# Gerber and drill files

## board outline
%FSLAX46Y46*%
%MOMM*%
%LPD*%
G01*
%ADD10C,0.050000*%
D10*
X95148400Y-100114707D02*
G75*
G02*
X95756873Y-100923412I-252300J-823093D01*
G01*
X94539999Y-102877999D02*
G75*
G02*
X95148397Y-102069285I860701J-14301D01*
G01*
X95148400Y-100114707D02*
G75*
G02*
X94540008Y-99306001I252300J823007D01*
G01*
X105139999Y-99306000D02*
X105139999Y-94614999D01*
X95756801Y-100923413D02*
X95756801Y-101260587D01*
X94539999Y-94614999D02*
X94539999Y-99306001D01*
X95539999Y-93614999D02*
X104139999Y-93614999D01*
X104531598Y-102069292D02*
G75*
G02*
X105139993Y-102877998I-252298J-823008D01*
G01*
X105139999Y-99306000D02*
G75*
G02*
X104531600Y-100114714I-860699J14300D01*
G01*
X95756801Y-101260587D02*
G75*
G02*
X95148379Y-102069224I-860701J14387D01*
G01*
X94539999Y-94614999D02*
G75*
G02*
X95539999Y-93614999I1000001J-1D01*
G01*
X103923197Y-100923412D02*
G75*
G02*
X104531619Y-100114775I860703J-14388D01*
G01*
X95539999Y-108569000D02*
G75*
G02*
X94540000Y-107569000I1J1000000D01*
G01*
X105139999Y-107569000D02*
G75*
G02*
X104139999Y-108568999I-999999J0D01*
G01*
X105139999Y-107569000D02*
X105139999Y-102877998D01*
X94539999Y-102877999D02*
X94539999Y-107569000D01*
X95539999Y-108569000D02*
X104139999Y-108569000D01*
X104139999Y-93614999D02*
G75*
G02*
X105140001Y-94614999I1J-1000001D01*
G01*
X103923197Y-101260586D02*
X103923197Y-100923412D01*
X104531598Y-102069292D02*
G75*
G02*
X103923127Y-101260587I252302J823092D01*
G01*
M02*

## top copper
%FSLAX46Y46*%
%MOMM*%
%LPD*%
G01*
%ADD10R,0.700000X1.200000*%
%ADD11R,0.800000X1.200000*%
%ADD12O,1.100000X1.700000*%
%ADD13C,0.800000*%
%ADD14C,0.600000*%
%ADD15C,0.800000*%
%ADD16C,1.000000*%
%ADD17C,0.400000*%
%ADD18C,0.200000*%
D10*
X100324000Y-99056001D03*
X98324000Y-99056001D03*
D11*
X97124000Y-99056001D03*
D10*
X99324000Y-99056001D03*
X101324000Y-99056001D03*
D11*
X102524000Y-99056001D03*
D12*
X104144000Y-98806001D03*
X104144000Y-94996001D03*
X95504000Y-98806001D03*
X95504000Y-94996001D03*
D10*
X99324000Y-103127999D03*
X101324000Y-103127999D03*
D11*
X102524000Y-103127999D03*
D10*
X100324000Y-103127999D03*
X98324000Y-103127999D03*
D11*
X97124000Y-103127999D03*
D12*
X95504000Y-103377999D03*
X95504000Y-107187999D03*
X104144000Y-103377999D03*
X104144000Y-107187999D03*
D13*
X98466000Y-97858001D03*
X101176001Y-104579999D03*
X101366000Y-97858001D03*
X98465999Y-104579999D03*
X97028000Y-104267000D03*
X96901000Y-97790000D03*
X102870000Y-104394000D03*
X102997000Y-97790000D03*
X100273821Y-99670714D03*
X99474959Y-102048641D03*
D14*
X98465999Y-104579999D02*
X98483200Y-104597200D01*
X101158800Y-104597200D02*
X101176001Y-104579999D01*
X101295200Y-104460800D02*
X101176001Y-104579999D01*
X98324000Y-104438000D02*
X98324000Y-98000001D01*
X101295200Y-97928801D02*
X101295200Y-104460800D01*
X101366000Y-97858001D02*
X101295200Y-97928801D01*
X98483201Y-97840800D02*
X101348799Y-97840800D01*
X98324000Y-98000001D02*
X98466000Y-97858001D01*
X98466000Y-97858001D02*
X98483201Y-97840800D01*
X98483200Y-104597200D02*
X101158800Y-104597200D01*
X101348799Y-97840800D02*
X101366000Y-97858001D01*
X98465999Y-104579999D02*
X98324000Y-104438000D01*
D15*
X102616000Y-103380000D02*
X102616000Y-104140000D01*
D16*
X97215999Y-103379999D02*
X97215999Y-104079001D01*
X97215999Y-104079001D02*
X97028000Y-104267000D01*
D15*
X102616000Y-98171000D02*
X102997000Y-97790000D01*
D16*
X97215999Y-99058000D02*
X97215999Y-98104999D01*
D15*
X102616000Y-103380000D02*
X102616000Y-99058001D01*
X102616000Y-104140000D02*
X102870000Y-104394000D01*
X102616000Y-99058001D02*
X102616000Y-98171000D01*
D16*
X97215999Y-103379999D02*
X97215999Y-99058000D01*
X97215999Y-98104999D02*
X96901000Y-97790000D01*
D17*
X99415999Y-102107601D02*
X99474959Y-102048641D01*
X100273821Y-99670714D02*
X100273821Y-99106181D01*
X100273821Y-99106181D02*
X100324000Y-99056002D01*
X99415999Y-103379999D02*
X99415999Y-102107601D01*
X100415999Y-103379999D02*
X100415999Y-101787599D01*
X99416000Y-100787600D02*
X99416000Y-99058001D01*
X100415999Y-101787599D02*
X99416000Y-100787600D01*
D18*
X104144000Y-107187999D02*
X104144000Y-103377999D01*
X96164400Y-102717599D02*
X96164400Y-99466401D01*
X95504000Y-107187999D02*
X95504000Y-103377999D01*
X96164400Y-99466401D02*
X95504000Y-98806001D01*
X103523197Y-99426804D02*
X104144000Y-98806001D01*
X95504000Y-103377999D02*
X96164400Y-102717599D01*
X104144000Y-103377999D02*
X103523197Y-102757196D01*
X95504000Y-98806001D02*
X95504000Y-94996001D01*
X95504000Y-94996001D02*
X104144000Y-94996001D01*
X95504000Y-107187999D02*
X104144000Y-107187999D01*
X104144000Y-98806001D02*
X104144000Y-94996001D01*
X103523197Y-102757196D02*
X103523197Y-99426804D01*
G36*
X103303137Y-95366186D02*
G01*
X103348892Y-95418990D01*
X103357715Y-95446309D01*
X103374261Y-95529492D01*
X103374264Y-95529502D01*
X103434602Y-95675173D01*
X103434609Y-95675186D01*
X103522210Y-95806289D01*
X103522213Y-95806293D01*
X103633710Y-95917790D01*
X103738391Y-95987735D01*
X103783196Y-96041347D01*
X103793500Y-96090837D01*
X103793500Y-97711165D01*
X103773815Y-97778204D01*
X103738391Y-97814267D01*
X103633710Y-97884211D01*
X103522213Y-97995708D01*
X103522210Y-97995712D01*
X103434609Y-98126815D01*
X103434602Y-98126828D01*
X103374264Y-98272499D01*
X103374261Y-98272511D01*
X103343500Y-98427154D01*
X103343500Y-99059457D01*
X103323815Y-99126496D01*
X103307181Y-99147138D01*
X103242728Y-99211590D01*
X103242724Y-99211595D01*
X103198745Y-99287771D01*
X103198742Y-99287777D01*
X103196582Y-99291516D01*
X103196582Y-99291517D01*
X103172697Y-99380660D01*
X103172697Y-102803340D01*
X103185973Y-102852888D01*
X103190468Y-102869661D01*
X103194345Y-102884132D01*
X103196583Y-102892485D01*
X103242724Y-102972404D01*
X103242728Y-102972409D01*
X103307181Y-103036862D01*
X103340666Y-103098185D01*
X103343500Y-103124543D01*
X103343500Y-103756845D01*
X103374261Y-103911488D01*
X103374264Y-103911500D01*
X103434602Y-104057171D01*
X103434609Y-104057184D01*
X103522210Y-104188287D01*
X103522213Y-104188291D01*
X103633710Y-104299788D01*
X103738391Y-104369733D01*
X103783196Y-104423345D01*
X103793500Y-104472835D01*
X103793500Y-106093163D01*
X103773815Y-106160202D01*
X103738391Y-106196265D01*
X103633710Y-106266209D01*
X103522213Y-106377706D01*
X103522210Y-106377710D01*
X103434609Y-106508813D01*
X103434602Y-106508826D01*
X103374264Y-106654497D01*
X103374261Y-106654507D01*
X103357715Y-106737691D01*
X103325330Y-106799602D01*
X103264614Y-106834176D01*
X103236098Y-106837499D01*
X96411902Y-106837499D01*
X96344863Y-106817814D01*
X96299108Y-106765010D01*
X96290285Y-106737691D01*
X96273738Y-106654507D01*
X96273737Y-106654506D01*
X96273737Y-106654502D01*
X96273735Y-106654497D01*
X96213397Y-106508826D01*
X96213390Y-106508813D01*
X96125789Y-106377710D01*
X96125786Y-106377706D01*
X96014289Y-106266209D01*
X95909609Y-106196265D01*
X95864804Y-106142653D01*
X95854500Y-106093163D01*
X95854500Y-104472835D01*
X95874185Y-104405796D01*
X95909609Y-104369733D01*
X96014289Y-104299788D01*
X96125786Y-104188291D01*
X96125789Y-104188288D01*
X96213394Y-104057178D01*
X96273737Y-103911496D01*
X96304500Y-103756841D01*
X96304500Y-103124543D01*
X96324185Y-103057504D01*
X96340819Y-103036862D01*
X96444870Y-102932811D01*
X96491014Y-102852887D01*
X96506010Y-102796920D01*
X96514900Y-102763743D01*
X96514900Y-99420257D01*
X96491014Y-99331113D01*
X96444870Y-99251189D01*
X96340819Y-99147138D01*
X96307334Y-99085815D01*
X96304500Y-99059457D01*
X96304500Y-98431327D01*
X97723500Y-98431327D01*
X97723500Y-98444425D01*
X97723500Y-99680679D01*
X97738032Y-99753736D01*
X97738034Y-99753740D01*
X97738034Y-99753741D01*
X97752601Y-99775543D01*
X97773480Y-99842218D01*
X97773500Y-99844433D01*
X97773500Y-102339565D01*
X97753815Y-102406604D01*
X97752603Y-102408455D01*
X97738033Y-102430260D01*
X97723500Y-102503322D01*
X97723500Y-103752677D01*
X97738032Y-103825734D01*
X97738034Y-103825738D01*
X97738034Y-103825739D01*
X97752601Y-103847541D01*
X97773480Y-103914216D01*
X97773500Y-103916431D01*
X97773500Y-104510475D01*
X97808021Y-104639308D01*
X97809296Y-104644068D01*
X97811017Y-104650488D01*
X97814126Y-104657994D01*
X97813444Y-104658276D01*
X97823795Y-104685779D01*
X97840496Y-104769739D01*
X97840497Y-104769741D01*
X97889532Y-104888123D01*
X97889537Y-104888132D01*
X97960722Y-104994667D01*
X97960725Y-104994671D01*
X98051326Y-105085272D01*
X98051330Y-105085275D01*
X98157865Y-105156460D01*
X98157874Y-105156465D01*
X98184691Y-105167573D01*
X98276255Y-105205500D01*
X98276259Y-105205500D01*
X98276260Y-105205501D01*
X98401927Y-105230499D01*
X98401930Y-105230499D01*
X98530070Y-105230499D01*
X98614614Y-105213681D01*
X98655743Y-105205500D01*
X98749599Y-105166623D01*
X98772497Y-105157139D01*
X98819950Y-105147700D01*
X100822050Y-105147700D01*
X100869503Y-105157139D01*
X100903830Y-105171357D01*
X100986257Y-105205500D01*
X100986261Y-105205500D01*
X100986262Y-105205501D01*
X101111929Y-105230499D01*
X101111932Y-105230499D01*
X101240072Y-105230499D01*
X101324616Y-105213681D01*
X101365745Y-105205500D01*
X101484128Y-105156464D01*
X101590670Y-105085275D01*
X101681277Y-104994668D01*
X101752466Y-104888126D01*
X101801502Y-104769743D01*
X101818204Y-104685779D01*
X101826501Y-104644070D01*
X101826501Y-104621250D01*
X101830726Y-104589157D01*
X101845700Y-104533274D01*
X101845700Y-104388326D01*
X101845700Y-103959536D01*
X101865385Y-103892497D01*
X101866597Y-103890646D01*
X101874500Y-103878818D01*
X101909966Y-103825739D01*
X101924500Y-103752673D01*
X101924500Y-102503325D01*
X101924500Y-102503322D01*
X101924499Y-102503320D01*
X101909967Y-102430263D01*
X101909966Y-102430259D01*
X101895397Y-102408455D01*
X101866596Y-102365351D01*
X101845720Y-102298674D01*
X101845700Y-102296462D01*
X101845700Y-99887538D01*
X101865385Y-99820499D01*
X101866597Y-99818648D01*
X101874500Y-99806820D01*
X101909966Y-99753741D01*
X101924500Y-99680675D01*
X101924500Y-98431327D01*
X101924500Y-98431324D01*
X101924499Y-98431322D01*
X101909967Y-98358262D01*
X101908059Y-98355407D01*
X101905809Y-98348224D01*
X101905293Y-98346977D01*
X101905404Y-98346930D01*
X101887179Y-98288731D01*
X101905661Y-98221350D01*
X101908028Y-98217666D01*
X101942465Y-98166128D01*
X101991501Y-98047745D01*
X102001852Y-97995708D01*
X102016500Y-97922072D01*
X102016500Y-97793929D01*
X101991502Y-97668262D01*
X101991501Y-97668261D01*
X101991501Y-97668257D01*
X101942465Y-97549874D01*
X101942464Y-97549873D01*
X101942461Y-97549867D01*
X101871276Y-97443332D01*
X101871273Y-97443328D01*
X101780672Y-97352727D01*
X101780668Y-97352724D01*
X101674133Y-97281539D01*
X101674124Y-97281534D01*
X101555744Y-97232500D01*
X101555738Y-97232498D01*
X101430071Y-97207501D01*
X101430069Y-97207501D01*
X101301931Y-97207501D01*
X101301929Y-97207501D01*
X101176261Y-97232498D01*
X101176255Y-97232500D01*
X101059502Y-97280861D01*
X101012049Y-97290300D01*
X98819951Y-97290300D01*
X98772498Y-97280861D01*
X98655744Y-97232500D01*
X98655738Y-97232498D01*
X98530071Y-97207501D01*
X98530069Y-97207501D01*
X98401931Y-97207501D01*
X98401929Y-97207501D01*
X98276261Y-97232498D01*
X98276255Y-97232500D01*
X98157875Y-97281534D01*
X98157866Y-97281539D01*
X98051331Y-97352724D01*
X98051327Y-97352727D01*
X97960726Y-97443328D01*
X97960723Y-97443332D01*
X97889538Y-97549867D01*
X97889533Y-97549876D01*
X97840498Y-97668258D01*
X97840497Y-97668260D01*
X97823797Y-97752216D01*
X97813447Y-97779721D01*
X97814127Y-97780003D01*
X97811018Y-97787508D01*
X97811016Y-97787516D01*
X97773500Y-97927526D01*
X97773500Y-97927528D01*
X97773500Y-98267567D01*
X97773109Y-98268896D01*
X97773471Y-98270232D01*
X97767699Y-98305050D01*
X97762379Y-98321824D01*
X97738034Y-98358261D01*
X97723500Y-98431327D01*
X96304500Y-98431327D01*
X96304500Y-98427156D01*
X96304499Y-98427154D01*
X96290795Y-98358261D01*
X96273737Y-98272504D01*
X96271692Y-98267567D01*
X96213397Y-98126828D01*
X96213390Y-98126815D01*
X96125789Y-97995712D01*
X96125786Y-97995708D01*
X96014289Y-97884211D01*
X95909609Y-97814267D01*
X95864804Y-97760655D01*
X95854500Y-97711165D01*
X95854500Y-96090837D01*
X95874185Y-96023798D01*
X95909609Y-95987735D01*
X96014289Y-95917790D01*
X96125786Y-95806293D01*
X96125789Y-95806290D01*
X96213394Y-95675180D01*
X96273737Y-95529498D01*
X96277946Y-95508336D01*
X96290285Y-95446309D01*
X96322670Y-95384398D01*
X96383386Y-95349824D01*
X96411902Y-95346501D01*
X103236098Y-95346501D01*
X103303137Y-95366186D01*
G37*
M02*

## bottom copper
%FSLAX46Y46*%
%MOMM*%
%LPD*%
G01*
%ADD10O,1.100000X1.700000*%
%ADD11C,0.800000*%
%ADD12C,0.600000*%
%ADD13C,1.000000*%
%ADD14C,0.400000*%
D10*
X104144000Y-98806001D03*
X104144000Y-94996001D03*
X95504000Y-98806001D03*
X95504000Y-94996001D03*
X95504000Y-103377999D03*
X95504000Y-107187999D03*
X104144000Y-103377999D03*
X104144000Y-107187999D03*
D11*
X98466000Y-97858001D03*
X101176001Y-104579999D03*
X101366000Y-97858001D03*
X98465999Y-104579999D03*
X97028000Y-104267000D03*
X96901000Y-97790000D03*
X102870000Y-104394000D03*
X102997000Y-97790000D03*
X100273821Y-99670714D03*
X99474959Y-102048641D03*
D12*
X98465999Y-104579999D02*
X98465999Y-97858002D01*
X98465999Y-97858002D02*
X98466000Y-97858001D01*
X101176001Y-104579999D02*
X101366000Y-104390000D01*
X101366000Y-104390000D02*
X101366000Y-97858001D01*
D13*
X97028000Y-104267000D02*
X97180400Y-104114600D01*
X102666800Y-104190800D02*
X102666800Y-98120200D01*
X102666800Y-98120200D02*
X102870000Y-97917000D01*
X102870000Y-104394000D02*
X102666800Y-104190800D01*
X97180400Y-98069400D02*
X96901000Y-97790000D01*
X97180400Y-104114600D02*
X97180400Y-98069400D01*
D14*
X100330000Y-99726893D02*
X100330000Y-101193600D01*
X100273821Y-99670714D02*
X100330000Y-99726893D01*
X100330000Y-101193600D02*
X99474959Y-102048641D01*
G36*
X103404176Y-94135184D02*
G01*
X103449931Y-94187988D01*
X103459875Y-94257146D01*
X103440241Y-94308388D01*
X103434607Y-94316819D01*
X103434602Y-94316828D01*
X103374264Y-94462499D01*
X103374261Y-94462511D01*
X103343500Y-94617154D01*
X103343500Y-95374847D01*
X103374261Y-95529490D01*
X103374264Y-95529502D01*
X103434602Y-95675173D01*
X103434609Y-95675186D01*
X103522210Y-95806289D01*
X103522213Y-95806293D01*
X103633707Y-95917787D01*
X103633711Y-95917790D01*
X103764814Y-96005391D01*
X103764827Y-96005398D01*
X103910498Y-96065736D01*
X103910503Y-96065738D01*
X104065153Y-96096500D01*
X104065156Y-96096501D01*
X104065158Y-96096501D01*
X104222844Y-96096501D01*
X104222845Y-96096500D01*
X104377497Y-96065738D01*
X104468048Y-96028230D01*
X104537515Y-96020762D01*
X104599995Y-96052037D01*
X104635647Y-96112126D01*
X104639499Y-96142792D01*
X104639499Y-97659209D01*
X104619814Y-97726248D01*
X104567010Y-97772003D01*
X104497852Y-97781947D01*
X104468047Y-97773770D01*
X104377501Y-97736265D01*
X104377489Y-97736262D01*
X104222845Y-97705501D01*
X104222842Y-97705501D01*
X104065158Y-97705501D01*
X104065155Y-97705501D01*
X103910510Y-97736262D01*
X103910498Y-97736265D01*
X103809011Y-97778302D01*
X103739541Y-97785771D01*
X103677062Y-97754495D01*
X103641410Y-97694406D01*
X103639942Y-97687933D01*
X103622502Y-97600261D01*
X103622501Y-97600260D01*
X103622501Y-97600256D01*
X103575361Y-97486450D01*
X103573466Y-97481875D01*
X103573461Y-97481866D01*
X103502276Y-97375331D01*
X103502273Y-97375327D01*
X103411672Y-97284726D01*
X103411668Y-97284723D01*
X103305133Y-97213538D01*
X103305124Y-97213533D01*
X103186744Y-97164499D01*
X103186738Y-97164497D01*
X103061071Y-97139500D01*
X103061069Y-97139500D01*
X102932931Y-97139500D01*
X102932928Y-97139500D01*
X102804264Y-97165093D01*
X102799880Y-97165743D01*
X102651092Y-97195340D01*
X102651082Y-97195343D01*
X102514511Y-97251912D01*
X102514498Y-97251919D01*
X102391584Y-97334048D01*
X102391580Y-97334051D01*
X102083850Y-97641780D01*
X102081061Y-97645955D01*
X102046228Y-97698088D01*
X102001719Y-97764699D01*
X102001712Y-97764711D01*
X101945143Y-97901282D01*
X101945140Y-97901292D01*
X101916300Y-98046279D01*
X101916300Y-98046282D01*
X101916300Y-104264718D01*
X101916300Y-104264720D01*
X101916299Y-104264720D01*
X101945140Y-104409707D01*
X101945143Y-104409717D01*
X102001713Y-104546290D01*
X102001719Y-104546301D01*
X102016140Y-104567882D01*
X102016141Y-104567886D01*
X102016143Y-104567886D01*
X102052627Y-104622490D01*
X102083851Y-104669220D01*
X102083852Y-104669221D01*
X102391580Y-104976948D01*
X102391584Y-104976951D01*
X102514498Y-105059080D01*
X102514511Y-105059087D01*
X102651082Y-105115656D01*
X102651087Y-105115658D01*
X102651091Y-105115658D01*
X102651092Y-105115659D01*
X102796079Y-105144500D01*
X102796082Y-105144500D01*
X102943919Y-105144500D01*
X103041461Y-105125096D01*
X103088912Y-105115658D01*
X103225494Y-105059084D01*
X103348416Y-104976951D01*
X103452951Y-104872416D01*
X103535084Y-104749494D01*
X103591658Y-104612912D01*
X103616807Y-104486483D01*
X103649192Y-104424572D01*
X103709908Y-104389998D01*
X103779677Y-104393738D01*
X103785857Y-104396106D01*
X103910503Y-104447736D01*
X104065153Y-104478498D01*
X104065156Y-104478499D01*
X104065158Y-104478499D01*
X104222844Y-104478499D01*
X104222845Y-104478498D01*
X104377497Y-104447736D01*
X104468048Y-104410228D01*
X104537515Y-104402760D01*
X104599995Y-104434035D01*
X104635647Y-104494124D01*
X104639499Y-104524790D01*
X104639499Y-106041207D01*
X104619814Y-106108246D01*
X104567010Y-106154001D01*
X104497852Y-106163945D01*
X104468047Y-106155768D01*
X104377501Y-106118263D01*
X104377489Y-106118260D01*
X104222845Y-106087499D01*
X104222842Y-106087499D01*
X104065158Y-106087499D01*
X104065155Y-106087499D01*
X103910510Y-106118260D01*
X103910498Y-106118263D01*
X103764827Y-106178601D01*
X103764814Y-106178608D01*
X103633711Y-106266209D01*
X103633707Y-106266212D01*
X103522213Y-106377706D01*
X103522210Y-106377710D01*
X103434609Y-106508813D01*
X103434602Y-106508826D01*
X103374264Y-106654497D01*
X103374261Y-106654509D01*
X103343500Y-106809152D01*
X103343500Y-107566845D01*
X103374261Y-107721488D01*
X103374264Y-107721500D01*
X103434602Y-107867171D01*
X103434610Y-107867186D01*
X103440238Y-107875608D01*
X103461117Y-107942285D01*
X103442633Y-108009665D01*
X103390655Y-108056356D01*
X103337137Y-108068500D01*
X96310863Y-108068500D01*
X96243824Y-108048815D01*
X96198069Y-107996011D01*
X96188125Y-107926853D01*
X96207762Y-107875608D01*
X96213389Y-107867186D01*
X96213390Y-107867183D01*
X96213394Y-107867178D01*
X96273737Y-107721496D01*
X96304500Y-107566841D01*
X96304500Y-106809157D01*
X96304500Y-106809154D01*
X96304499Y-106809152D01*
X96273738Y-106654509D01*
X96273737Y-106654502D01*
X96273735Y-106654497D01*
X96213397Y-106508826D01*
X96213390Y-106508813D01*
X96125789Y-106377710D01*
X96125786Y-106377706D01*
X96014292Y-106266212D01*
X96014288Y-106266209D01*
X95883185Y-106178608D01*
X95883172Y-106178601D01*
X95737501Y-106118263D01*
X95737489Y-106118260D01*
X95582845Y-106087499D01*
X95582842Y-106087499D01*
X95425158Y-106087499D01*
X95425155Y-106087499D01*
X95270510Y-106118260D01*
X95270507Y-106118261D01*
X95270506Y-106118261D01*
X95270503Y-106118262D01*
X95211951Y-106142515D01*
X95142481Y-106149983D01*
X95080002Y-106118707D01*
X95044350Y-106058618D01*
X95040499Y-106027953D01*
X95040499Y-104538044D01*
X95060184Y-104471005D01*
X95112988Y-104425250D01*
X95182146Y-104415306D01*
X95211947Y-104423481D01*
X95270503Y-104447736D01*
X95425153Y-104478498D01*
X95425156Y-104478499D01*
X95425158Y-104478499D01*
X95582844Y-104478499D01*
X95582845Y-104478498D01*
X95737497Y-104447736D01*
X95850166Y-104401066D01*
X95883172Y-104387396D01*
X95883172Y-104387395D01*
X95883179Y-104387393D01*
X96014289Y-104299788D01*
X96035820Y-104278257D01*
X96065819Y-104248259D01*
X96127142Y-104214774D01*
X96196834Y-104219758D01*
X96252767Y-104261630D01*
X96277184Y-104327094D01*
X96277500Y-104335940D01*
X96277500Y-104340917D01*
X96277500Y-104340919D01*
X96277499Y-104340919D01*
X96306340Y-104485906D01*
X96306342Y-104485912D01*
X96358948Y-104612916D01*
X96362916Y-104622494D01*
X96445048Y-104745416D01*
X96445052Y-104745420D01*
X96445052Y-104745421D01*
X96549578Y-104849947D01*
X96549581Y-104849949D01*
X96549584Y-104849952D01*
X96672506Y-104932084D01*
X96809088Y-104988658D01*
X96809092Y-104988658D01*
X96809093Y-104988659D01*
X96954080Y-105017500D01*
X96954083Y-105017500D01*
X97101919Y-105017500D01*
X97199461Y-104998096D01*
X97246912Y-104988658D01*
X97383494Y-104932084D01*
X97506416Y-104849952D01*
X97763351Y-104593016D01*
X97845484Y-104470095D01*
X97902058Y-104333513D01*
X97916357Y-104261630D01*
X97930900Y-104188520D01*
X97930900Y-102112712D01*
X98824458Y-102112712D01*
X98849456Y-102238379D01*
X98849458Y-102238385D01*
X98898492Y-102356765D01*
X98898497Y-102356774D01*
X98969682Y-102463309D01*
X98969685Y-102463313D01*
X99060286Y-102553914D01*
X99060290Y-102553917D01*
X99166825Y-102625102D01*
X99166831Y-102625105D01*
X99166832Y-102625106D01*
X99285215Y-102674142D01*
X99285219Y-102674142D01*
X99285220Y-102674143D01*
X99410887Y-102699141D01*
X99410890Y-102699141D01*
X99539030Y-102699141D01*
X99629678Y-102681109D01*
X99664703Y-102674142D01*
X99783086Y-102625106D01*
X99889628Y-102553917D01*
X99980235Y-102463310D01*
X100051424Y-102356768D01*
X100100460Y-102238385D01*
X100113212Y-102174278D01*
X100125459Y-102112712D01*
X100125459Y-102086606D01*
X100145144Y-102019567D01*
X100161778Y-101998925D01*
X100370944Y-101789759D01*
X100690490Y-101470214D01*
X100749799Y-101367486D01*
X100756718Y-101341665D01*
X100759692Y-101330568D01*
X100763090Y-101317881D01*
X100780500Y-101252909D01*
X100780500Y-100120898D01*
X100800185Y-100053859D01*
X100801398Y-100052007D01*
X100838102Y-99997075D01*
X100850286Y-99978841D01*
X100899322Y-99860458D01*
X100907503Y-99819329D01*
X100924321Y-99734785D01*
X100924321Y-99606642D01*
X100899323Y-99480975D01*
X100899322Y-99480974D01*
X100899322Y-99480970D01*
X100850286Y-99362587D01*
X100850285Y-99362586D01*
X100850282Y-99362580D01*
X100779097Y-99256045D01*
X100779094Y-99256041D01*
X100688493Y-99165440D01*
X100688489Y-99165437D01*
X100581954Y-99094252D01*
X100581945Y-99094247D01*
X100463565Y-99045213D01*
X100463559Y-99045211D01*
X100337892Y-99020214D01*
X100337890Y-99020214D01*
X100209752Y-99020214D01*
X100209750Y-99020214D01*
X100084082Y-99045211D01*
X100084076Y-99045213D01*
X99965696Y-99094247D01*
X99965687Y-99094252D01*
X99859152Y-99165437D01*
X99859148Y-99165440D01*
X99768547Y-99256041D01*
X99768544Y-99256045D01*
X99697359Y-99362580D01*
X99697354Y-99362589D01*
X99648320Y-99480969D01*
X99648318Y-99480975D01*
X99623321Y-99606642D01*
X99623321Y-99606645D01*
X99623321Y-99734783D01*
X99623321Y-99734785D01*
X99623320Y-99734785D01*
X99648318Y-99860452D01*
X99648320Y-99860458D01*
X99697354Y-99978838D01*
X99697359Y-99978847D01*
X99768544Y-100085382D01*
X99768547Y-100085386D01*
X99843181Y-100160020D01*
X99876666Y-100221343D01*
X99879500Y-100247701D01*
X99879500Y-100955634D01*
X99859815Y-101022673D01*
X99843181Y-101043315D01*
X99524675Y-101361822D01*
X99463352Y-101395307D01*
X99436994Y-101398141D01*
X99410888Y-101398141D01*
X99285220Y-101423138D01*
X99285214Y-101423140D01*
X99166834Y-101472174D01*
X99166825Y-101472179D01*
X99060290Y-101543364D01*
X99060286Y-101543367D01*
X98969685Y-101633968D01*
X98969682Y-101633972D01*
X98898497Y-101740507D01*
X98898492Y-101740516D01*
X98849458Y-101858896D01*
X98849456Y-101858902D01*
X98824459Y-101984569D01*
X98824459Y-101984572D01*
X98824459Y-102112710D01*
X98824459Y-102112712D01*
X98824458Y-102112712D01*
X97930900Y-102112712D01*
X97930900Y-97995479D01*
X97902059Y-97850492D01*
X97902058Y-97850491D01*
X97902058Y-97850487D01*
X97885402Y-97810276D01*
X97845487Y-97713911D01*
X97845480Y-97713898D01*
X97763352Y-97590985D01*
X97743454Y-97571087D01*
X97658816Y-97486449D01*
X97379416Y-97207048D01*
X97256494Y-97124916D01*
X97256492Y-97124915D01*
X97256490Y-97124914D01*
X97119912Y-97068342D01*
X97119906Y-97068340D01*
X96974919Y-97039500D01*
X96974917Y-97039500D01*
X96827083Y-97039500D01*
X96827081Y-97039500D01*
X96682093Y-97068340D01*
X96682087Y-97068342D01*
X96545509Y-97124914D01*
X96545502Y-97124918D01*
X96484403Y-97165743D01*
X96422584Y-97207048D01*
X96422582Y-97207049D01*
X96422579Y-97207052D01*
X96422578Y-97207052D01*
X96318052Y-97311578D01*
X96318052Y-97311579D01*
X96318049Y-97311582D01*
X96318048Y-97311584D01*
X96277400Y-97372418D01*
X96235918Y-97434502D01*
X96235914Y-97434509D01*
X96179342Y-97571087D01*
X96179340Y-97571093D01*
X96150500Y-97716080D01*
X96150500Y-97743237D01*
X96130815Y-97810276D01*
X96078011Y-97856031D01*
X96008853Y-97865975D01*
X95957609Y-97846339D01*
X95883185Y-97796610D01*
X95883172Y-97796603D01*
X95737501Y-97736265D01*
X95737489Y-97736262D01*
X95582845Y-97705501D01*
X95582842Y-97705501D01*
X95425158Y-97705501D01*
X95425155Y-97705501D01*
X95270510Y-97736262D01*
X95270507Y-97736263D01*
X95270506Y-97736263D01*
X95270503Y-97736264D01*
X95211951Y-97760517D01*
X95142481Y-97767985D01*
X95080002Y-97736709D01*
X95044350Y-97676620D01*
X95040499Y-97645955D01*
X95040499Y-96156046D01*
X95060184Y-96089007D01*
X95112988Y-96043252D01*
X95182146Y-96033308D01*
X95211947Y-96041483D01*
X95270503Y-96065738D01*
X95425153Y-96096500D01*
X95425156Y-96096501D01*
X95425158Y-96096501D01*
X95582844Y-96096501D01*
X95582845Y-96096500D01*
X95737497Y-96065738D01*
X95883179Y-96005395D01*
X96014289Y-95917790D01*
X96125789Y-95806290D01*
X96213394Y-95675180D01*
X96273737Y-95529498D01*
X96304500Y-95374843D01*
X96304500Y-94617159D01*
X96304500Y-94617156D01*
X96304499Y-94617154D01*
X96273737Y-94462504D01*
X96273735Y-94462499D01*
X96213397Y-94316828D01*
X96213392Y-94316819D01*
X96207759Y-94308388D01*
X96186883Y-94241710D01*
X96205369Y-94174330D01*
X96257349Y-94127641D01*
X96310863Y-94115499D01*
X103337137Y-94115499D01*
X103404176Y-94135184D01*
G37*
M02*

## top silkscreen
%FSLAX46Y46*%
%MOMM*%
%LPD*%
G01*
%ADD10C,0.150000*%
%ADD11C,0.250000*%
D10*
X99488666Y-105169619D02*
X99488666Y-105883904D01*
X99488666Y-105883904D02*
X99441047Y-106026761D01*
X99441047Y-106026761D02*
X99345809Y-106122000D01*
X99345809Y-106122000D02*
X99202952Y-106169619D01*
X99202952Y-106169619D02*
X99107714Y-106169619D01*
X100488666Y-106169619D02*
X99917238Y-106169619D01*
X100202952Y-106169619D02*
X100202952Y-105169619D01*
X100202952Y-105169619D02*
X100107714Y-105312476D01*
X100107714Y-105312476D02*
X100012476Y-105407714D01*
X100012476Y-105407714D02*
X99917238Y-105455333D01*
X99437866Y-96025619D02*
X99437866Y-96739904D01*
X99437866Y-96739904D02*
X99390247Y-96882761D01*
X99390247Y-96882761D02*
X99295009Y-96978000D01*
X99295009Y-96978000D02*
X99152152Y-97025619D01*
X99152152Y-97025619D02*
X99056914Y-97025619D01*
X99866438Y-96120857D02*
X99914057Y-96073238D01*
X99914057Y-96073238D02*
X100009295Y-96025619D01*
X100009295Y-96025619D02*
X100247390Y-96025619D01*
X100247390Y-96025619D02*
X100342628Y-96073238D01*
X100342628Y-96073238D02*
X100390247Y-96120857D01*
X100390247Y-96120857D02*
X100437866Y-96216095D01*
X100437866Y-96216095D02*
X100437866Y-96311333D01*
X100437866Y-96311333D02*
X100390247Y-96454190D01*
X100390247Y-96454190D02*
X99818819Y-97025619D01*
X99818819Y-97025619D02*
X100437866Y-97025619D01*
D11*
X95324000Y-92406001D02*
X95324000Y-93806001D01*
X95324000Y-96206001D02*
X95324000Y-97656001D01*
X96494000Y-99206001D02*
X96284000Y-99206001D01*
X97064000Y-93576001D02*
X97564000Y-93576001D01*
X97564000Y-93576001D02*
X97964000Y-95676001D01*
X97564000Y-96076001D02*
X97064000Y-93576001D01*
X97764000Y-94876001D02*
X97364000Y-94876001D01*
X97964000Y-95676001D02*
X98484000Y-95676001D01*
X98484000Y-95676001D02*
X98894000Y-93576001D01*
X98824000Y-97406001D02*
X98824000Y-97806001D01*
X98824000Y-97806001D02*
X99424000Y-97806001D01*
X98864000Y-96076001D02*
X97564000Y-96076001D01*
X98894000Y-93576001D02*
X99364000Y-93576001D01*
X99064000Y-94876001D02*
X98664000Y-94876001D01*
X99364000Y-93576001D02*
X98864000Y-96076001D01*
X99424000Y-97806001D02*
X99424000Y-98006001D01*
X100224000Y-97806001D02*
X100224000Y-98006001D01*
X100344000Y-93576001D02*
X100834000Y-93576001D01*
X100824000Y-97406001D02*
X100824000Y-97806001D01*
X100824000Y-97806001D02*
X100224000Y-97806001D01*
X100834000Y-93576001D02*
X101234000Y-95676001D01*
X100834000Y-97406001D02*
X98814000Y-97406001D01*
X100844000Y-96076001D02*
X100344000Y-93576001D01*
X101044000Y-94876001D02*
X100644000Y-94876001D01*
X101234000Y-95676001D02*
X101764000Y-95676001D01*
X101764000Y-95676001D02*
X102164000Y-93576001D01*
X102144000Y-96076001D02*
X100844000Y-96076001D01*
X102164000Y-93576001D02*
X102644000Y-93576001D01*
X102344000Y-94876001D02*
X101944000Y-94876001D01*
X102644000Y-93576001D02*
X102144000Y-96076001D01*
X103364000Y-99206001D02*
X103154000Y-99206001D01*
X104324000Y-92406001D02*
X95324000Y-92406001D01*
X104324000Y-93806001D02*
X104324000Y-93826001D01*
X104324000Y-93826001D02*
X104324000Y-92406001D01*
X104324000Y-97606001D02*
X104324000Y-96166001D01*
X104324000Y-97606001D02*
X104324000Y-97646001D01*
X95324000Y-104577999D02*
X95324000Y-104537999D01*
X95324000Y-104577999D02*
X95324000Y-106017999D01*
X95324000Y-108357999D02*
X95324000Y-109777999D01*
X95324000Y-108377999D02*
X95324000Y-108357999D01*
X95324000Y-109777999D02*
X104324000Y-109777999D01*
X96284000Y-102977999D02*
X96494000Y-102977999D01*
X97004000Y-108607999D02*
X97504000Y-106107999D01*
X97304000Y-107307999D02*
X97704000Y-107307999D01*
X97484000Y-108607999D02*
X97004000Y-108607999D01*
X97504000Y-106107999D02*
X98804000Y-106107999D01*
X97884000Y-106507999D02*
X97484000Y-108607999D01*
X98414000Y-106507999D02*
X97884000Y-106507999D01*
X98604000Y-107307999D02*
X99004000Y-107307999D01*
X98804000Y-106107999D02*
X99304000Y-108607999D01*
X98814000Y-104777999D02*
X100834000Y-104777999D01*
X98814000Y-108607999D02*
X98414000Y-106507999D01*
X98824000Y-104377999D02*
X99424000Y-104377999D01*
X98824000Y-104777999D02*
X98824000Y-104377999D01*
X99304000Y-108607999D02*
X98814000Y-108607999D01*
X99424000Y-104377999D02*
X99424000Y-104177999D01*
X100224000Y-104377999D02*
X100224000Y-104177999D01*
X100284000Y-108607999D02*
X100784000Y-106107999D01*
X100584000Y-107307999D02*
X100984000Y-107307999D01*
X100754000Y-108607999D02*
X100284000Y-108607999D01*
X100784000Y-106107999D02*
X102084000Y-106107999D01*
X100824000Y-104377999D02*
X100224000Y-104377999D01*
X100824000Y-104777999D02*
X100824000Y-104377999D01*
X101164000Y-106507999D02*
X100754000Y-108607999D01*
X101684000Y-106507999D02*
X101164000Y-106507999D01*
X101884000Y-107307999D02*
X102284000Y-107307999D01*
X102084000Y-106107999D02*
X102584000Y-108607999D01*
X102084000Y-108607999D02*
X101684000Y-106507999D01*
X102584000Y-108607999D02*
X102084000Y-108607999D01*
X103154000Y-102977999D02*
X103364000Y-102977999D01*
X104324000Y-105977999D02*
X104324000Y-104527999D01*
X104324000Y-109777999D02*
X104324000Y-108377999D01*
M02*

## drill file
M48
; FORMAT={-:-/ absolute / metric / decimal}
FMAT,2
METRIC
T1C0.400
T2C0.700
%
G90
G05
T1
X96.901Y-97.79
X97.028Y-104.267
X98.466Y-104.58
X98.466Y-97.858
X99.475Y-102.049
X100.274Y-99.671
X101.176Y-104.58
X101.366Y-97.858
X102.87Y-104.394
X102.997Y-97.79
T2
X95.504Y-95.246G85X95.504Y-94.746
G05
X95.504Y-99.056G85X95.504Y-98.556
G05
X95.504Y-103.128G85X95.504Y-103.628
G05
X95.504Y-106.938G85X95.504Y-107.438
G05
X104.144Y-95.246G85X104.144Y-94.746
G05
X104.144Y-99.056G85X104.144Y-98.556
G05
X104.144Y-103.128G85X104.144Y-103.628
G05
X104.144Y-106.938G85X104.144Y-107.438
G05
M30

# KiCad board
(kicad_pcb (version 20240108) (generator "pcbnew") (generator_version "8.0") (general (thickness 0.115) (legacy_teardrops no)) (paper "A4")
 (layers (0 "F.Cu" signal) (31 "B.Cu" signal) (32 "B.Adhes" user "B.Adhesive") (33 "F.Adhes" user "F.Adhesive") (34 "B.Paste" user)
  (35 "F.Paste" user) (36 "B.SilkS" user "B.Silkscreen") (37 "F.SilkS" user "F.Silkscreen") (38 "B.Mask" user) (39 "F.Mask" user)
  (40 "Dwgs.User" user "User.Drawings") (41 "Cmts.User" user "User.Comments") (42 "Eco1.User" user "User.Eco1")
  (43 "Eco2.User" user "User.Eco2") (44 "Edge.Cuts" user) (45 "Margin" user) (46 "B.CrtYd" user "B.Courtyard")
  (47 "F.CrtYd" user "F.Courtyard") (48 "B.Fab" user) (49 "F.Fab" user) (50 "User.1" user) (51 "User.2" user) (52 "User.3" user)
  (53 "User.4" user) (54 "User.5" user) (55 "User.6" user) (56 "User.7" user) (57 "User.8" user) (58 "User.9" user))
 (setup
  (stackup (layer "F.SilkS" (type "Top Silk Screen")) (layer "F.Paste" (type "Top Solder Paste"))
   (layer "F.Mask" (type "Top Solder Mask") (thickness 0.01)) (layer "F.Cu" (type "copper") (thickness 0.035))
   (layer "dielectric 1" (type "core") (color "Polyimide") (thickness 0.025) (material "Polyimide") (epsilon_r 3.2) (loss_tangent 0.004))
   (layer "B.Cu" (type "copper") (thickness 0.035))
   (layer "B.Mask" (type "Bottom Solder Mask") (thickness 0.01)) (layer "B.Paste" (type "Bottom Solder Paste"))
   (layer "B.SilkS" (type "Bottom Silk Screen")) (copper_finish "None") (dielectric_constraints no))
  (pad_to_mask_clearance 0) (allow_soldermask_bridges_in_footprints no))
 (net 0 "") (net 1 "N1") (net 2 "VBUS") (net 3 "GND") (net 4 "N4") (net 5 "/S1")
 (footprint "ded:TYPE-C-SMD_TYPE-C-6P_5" (layer "F.Cu") (at 99.824 97.026001 180)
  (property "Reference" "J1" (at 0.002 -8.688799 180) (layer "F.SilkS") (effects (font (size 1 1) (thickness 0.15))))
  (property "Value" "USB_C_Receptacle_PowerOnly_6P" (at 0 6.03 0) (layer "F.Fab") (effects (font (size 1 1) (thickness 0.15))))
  (fp_line (start 4.5 4.62) (end 4.5 3.22) (stroke (width 0.25) (type solid)) (layer "F.SilkS"))
  (fp_line (start 4.5 0.82) (end 4.5 -0.63) (stroke (width 0.25) (type solid)) (layer "F.SilkS"))
  (fp_line (start 3.33 -2.18) (end 3.54 -2.18) (stroke (width 0.25) (type solid)) (layer "F.SilkS"))
  (fp_line (start 2.76 3.45) (end 2.26 3.45) (stroke (width 0.25) (type solid)) (layer "F.SilkS"))
  (fp_line (start 2.26 3.45) (end 1.86 1.35) (stroke (width 0.25) (type solid)) (layer "F.SilkS"))
  (fp_line (start 2.26 0.95) (end 2.76 3.45) (stroke (width 0.25) (type solid)) (layer "F.SilkS"))
  (fp_line (start 2.06 2.15) (end 2.46 2.15) (stroke (width 0.25) (type solid)) (layer "F.SilkS"))
  (fp_line (start 1.86 1.35) (end 1.34 1.35) (stroke (width 0.25) (type solid)) (layer "F.SilkS"))
  (fp_line (start 1.34 1.35) (end 0.93 3.45) (stroke (width 0.25) (type solid)) (layer "F.SilkS"))
  (fp_line (start 1 -0.38) (end 1 -0.78) (stroke (width 0.25) (type solid)) (layer "F.SilkS"))
  (fp_line (start 1 -0.78) (end 0.4 -0.78) (stroke (width 0.25) (type solid)) (layer "F.SilkS"))
  (fp_line (start 0.96 0.95) (end 2.26 0.95) (stroke (width 0.25) (type solid)) (layer "F.SilkS"))
  (fp_line (start 0.93 3.45) (end 0.46 3.45) (stroke (width 0.25) (type solid)) (layer "F.SilkS"))
  (fp_line (start 0.76 2.15) (end 1.16 2.15) (stroke (width 0.25) (type solid)) (layer "F.SilkS"))
  (fp_line (start 0.46 3.45) (end 0.96 0.95) (stroke (width 0.25) (type solid)) (layer "F.SilkS"))
  (fp_line (start 0.4 -0.78) (end 0.4 -0.98) (stroke (width 0.25) (type solid)) (layer "F.SilkS"))
  (fp_line (start -0.4 -0.78) (end -0.4 -0.98) (stroke (width 0.25) (type solid)) (layer "F.SilkS"))
  (fp_line (start -0.52 3.45) (end -1.01 3.45) (stroke (width 0.25) (type solid)) (layer "F.SilkS"))
  (fp_line (start -1 -0.38) (end -1 -0.78) (stroke (width 0.25) (type solid)) (layer "F.SilkS"))
  (fp_line (start -1 -0.78) (end -0.4 -0.78) (stroke (width 0.25) (type solid)) (layer "F.SilkS"))
  (fp_line (start -1.01 3.45) (end -1.41 1.35) (stroke (width 0.25) (type solid)) (layer "F.SilkS"))
  (fp_line (start -1.01 -0.38) (end 1.01 -0.38) (stroke (width 0.25) (type solid)) (layer "F.SilkS"))
  (fp_line (start -1.02 0.95) (end -0.52 3.45) (stroke (width 0.25) (type solid)) (layer "F.SilkS"))
  (fp_line (start -1.22 2.15) (end -0.82 2.15) (stroke (width 0.25) (type solid)) (layer "F.SilkS"))
  (fp_line (start -1.41 1.35) (end -1.94 1.35) (stroke (width 0.25) (type solid)) (layer "F.SilkS"))
  (fp_line (start -1.94 1.35) (end -2.34 3.45) (stroke (width 0.25) (type solid)) (layer "F.SilkS"))
  (fp_line (start -2.32 0.95) (end -1.02 0.95) (stroke (width 0.25) (type solid)) (layer "F.SilkS"))
  (fp_line (start -2.34 3.45) (end -2.82 3.45) (stroke (width 0.25) (type solid)) (layer "F.SilkS"))
  (fp_line (start -2.52 2.15) (end -2.12 2.15) (stroke (width 0.25) (type solid)) (layer "F.SilkS"))
  (fp_line (start -2.82 3.45) (end -2.32 0.95) (stroke (width 0.25) (type solid)) (layer "F.SilkS"))
  (fp_line (start -3.54 -2.18) (end -3.33 -2.18) (stroke (width 0.25) (type solid)) (layer "F.SilkS"))
  (fp_line (start -4.5 4.62) (end 4.5 4.62) (stroke (width 0.25) (type solid)) (layer "F.SilkS"))
  (fp_line (start -4.5 3.22) (end -4.5 3.2) (stroke (width 0.25) (type solid)) (layer "F.SilkS"))
  (fp_line (start -4.5 3.2) (end -4.5 4.62) (stroke (width 0.25) (type solid)) (layer "F.SilkS"))
  (fp_line (start -4.5 -0.58) (end -4.5 0.86) (stroke (width 0.25) (type solid)) (layer "F.SilkS"))
  (fp_line (start -4.5 -0.58) (end -4.5 -0.62) (stroke (width 0.25) (type solid)) (layer "F.SilkS"))
  (pad "A5" smd rect (at -0.5 -2.03 180) (size 0.7 1.2) (layers "F.Cu" "F.Paste" "F.Mask") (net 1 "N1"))
  (pad "A9" smd rect (at 1.5 -2.03 180) (size 0.7 1.2) (layers "F.Cu" "F.Paste" "F.Mask") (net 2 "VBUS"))
  (pad "A12" smd rect (at 2.7 -2.03 180) (size 0.8 1.2) (layers "F.Cu" "F.Paste" "F.Mask") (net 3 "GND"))
  (pad "B5" smd rect (at 0.5 -2.03 180) (size 0.7 1.2) (layers "F.Cu" "F.Paste" "F.Mask") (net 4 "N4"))
  (pad "B9" smd rect (at -1.5 -2.03 180) (size 0.7 1.2) (layers "F.Cu" "F.Paste" "F.Mask") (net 2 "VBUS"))
  (pad "B12" smd rect (at -2.7 -2.03 180) (size 0.8 1.2) (layers "F.Cu" "F.Paste" "F.Mask") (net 3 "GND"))
  (pad "S1" thru_hole oval (at -4.32 -1.78 180) (size 1.1 1.7) (drill oval 0.700024 1.199998) (layers "*.Cu" "*.Mask")
   (remove_unused_layers no) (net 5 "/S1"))
  (pad "S1" thru_hole oval (at -4.32 2.03 180) (size 1.1 1.7) (drill oval 0.700024 1.199998) (layers "*.Cu" "*.Mask")
   (remove_unused_layers no) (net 5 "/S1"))
  (pad "S1" thru_hole oval (at 4.32 -1.78 180) (size 1.1 1.7) (drill oval 0.700024 1.199998) (layers "*.Cu" "*.Mask")
   (remove_unused_layers no) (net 5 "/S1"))
  (pad "S1" thru_hole oval (at 4.32 2.03 180) (size 1.1 1.7) (drill oval 0.700024 1.199998) (layers "*.Cu" "*.Mask")
   (remove_unused_layers no) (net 5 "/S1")))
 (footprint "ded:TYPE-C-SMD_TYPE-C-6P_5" (layer "F.Cu") (at 99.824 105.157999)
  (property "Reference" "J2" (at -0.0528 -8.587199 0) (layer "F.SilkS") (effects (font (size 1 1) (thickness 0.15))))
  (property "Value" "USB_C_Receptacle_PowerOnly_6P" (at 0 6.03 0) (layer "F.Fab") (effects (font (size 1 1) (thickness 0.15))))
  (fp_line (start -4.5 -0.58) (end -4.5 -0.62) (stroke (width 0.25) (type solid)) (layer "F.SilkS"))
  (fp_line (start -4.5 -0.58) (end -4.5 0.86) (stroke (width 0.25) (type solid)) (layer "F.SilkS"))
  (fp_line (start -4.5 3.2) (end -4.5 4.62) (stroke (width 0.25) (type solid)) (layer "F.SilkS"))
  (fp_line (start -4.5 3.22) (end -4.5 3.2) (stroke (width 0.25) (type solid)) (layer "F.SilkS"))
  (fp_line (start -4.5 4.62) (end 4.5 4.62) (stroke (width 0.25) (type solid)) (layer "F.SilkS"))
  (fp_line (start -3.54 -2.18) (end -3.33 -2.18) (stroke (width 0.25) (type solid)) (layer "F.SilkS"))
  (fp_line (start -2.82 3.45) (end -2.32 0.95) (stroke (width 0.25) (type solid)) (layer "F.SilkS"))
  (fp_line (start -2.52 2.15) (end -2.12 2.15) (stroke (width 0.25) (type solid)) (layer "F.SilkS"))
  (fp_line (start -2.34 3.45) (end -2.82 3.45) (stroke (width 0.25) (type solid)) (layer "F.SilkS"))
  (fp_line (start -2.32 0.95) (end -1.02 0.95) (stroke (width 0.25) (type solid)) (layer "F.SilkS"))
  (fp_line (start -1.94 1.35) (end -2.34 3.45) (stroke (width 0.25) (type solid)) (layer "F.SilkS"))
  (fp_line (start -1.41 1.35) (end -1.94 1.35) (stroke (width 0.25) (type solid)) (layer "F.SilkS"))
  (fp_line (start -1.22 2.15) (end -0.82 2.15) (stroke (width 0.25) (type solid)) (layer "F.SilkS"))
  (fp_line (start -1.02 0.95) (end -0.52 3.45) (stroke (width 0.25) (type solid)) (layer "F.SilkS"))
  (fp_line (start -1.01 -0.38) (end 1.01 -0.38) (stroke (width 0.25) (type solid)) (layer "F.SilkS"))
  (fp_line (start -1.01 3.45) (end -1.41 1.35) (stroke (width 0.25) (type solid)) (layer "F.SilkS"))
  (fp_line (start -1 -0.78) (end -0.4 -0.78) (stroke (width 0.25) (type solid)) (layer "F.SilkS"))
  (fp_line (start -1 -0.38) (end -1 -0.78) (stroke (width 0.25) (type solid)) (layer "F.SilkS"))
  (fp_line (start -0.52 3.45) (end -1.01 3.45) (stroke (width 0.25) (type solid)) (layer "F.SilkS"))
  (fp_line (start -0.4 -0.78) (end -0.4 -0.98) (stroke (width 0.25) (type solid)) (layer "F.SilkS"))
  (fp_line (start 0.4 -0.78) (end 0.4 -0.98) (stroke (width 0.25) (type solid)) (layer "F.SilkS"))
  (fp_line (start 0.46 3.45) (end 0.96 0.95) (stroke (width 0.25) (type solid)) (layer "F.SilkS"))
  (fp_line (start 0.76 2.15) (end 1.16 2.15) (stroke (width 0.25) (type solid)) (layer "F.SilkS"))
  (fp_line (start 0.93 3.45) (end 0.46 3.45) (stroke (width 0.25) (type solid)) (layer "F.SilkS"))
  (fp_line (start 0.96 0.95) (end 2.26 0.95) (stroke (width 0.25) (type solid)) (layer "F.SilkS"))
  (fp_line (start 1 -0.78) (end 0.4 -0.78) (stroke (width 0.25) (type solid)) (layer "F.SilkS"))
  (fp_line (start 1 -0.38) (end 1 -0.78) (stroke (width 0.25) (type solid)) (layer "F.SilkS"))
  (fp_line (start 1.34 1.35) (end 0.93 3.45) (stroke (width 0.25) (type solid)) (layer "F.SilkS"))
  (fp_line (start 1.86 1.35) (end 1.34 1.35) (stroke (width 0.25) (type solid)) (layer "F.SilkS"))
  (fp_line (start 2.06 2.15) (end 2.46 2.15) (stroke (width 0.25) (type solid)) (layer "F.SilkS"))
  (fp_line (start 2.26 0.95) (end 2.76 3.45) (stroke (width 0.25) (type solid)) (layer "F.SilkS"))
  (fp_line (start 2.26 3.45) (end 1.86 1.35) (stroke (width 0.25) (type solid)) (layer "F.SilkS"))
  (fp_line (start 2.76 3.45) (end 2.26 3.45) (stroke (width 0.25) (type solid)) (layer "F.SilkS"))
  (fp_line (start 3.33 -2.18) (end 3.54 -2.18) (stroke (width 0.25) (type solid)) (layer "F.SilkS"))
  (fp_line (start 4.5 0.82) (end 4.5 -0.63) (stroke (width 0.25) (type solid)) (layer "F.SilkS"))
  (fp_line (start 4.5 4.62) (end 4.5 3.22) (stroke (width 0.25) (type solid)) (layer "F.SilkS"))
  (pad "A5" smd rect (at -0.5 -2.03) (size 0.7 1.2) (layers "F.Cu" "F.Paste" "F.Mask") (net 1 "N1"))
  (pad "A9" smd rect (at 1.5 -2.03) (size 0.7 1.2) (layers "F.Cu" "F.Paste" "F.Mask") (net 2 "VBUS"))
  (pad "A12" smd rect (at 2.7 -2.03) (size 0.8 1.2) (layers "F.Cu" "F.Paste" "F.Mask") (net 3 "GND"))
  (pad "B5" smd rect (at 0.5 -2.03) (size 0.7 1.2) (layers "F.Cu" "F.Paste" "F.Mask") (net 4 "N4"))
  (pad "B9" smd rect (at -1.5 -2.03) (size 0.7 1.2) (layers "F.Cu" "F.Paste" "F.Mask") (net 2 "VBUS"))
  (pad "B12" smd rect (at -2.7 -2.03) (size 0.8 1.2) (layers "F.Cu" "F.Paste" "F.Mask") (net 3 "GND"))
  (pad "S1" thru_hole oval (at -4.32 -1.78) (size 1.1 1.7) (drill oval 0.700024 1.199998) (layers "*.Cu" "*.Mask") (remove_unused_layers no)
   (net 5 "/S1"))
  (pad "S1" thru_hole oval (at -4.32 2.03) (size 1.1 1.7) (drill oval 0.700024 1.199998) (layers "*.Cu" "*.Mask") (remove_unused_layers no)
   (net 5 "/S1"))
  (pad "S1" thru_hole oval (at 4.32 -1.78) (size 1.1 1.7) (drill oval 0.700024 1.199998) (layers "*.Cu" "*.Mask") (remove_unused_layers no)
   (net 5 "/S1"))
  (pad "S1" thru_hole oval (at 4.32 2.03) (size 1.1 1.7) (drill oval 0.700024 1.199998) (layers "*.Cu" "*.Mask") (remove_unused_layers no)
   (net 5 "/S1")))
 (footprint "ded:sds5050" (layer "B.Cu") (at 100 101.092 180)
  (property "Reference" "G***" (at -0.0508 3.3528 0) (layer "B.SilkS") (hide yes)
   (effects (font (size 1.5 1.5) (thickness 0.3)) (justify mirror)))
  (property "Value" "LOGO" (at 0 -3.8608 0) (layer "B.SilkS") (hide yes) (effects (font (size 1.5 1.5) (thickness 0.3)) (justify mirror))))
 (gr_arc (start 95.1484 100.114707) (mid 95.583983 100.420219) (end 95.756801 100.923413) (stroke (width 0.05) (type default))
  (layer "Edge.Cuts"))
 (gr_arc (start 94.539999 102.877999) (mid 94.712817 102.374805) (end 95.1484 102.069293) (stroke (width 0.05) (type default))
  (layer "Edge.Cuts"))
 (gr_arc (start 95.1484 100.114707) (mid 94.712817 99.809195) (end 94.539999 99.306001) (stroke (width 0.05) (type default))
  (layer "Edge.Cuts"))
 (gr_line (start 105.139999 99.306) (end 105.139999 94.614999) (stroke (width 0.05) (type default)) (layer "Edge.Cuts"))
 (gr_line (start 95.756801 100.923413) (end 95.756801 101.260587) (stroke (width 0.05) (type default)) (layer "Edge.Cuts"))
 (gr_line (start 94.539999 94.614999) (end 94.539999 99.306001) (stroke (width 0.05) (type default)) (layer "Edge.Cuts"))
 (gr_line (start 95.539999 93.614999) (end 104.139999 93.614999) (stroke (width 0.05) (type default)) (layer "Edge.Cuts"))
 (gr_arc (start 104.531598 102.069292) (mid 104.967181 102.374804) (end 105.139999 102.877998) (stroke (width 0.05) (type default))
  (layer "Edge.Cuts"))
 (gr_arc (start 105.139999 99.306) (mid 104.967181 99.809194) (end 104.531598 100.114706) (stroke (width 0.05) (type default))
  (layer "Edge.Cuts"))
 (gr_arc (start 95.756801 101.260587) (mid 95.583983 101.763781) (end 95.1484 102.069293) (stroke (width 0.05) (type default))
  (layer "Edge.Cuts"))
 (gr_arc (start 94.539999 94.614999) (mid 94.832892 93.907892) (end 95.539999 93.614999) (stroke (width 0.05) (type default))
  (layer "Edge.Cuts"))
 (gr_arc (start 103.923197 100.923412) (mid 104.096015 100.420218) (end 104.531598 100.114706) (stroke (width 0.05) (type default))
  (layer "Edge.Cuts"))
 (gr_arc (start 95.539999 108.569) (mid 94.832892 108.276107) (end 94.539999 107.569) (stroke (width 0.05) (type default))
  (layer "Edge.Cuts"))
 (gr_arc (start 105.139999 107.569) (mid 104.847106 108.276107) (end 104.139999 108.569) (stroke (width 0.05) (type default))
  (layer "Edge.Cuts"))
 (gr_line (start 105.139999 107.569) (end 105.139999 102.877998) (stroke (width 0.05) (type default)) (layer "Edge.Cuts"))
 (gr_line (start 94.539999 102.877999) (end 94.539999 107.569) (stroke (width 0.05) (type default)) (layer "Edge.Cuts"))
 (gr_line (start 95.539999 108.569) (end 104.139999 108.569) (stroke (width 0.05) (type default)) (layer "Edge.Cuts"))
 (gr_arc (start 104.139999 93.614999) (mid 104.847106 93.907892) (end 105.139999 94.614999) (stroke (width 0.05) (type default))
  (layer "Edge.Cuts"))
 (gr_line (start 103.923197 101.260586) (end 103.923197 100.923412) (stroke (width 0.05) (type default)) (layer "Edge.Cuts"))
 (gr_arc (start 104.531598 102.069292) (mid 104.096015 101.76378) (end 103.923197 101.260586) (stroke (width 0.05) (type default))
  (layer "Edge.Cuts"))
 (segment (start 98.465999 104.579999) (end 98.4832 104.5972) (width 0.6) (layer "F.Cu") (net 2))
 (segment (start 101.1588 104.5972) (end 101.176001 104.579999) (width 0.6) (layer "F.Cu") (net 2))
 (segment (start 101.2952 104.4608) (end 101.176001 104.579999) (width 0.6) (layer "F.Cu") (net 2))
 (segment (start 98.324 104.438) (end 98.324 98.000001) (width 0.6) (layer "F.Cu") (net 2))
 (segment (start 101.2952 97.928801) (end 101.2952 104.4608) (width 0.6) (layer "F.Cu") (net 2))
 (segment (start 101.366 97.858001) (end 101.2952 97.928801) (width 0.6) (layer "F.Cu") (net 2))
 (segment (start 98.483201 97.8408) (end 101.348799 97.8408) (width 0.6) (layer "F.Cu") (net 2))
 (segment (start 98.324 98.000001) (end 98.466 97.858001) (width 0.6) (layer "F.Cu") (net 2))
 (segment (start 98.466 97.858001) (end 98.483201 97.8408) (width 0.6) (layer "F.Cu") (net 2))
 (segment (start 98.4832 104.5972) (end 101.1588 104.5972) (width 0.6) (layer "F.Cu") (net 2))
 (segment (start 101.348799 97.8408) (end 101.366 97.858001) (width 0.6) (layer "F.Cu") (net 2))
 (segment (start 98.465999 104.579999) (end 98.324 104.438) (width 0.6) (layer "F.Cu") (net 2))
 (via (at 98.466 97.858001) (size 0.8) (drill 0.4) (layers "F.Cu" "B.Cu") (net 2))
 (via (at 101.176001 104.579999) (size 0.8) (drill 0.4) (layers "F.Cu" "B.Cu") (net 2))
 (via (at 101.366 97.858001) (size 0.8) (drill 0.4) (layers "F.Cu" "B.Cu") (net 2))
 (via (at 98.465999 104.579999) (size 0.8) (drill 0.4) (layers "F.Cu" "B.Cu") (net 2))
 (segment (start 98.465999 104.579999) (end 98.465999 97.858002) (width 0.6) (layer "B.Cu") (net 2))
 (segment (start 98.465999 97.858002) (end 98.466 97.858001) (width 0.6) (layer "B.Cu") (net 2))
 (segment (start 101.176001 104.579999) (end 101.366 104.39) (width 0.6) (layer "B.Cu") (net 2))
 (segment (start 101.366 104.39) (end 101.366 97.858001) (width 0.6) (layer "B.Cu") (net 2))
 (segment (start 102.616 103.38) (end 102.616 104.14) (width 0.8) (layer "F.Cu") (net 3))
 (segment (start 97.215999 103.379999) (end 97.215999 104.079001) (width 1) (layer "F.Cu") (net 3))
 (segment (start 97.215999 104.079001) (end 97.028 104.267) (width 1) (layer "F.Cu") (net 3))
 (segment (start 102.616 98.171) (end 102.997 97.79) (width 0.8) (layer "F.Cu") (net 3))
 (segment (start 97.215999 99.058) (end 97.215999 98.104999) (width 1) (layer "F.Cu") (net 3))
 (segment (start 102.616 103.38) (end 102.616 99.058001) (width 0.8) (layer "F.Cu") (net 3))
 (segment (start 102.616 104.14) (end 102.87 104.394) (width 0.8) (layer "F.Cu") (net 3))
 (segment (start 102.616 99.058001) (end 102.616 98.171) (width 0.8) (layer "F.Cu") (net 3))
 (segment (start 97.215999 103.379999) (end 97.215999 99.058) (width 1) (layer "F.Cu") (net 3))
 (segment (start 97.215999 98.104999) (end 96.901 97.79) (width 1) (layer "F.Cu") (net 3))
 (via (at 97.028 104.267) (size 0.8) (drill 0.4) (layers "F.Cu" "B.Cu") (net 3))
 (via (at 96.901 97.79) (size 0.8) (drill 0.4) (layers "F.Cu" "B.Cu") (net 3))
 (via (at 102.87 104.394) (size 0.8) (drill 0.4) (layers "F.Cu" "B.Cu") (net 3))
 (via (at 102.997 97.79) (size 0.8) (drill 0.4) (layers "F.Cu" "B.Cu") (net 3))
 (segment (start 97.028 104.267) (end 97.1804 104.1146) (width 1) (layer "B.Cu") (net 3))
 (segment (start 102.6668 104.1908) (end 102.6668 98.1202) (width 1) (layer "B.Cu") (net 3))
 (segment (start 102.6668 98.1202) (end 102.87 97.917) (width 1) (layer "B.Cu") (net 3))
 (segment (start 102.87 104.394) (end 102.6668 104.1908) (width 1) (layer "B.Cu") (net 3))
 (segment (start 97.1804 98.0694) (end 96.901 97.79) (width 1) (layer "B.Cu") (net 3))
 (segment (start 97.1804 104.1146) (end 97.1804 98.0694) (width 1) (layer "B.Cu") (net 3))
 (segment (start 99.415999 102.107601) (end 99.474959 102.048641) (width 0.4) (layer "F.Cu") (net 1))
 (segment (start 100.273821 99.670714) (end 100.273821 99.106181) (width 0.4) (layer "F.Cu") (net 1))
 (segment (start 100.273821 99.106181) (end 100.324 99.056002) (width 0.4) (layer "F.Cu") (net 1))
 (segment (start 99.415999 103.379999) (end 99.415999 102.107601) (width 0.4) (layer "F.Cu") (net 1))
 (via (at 100.273821 99.670714) (size 0.8) (drill 0.4) (layers "F.Cu" "B.Cu") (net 1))
 (via (at 99.474959 102.048641) (size 0.8) (drill 0.4) (layers "F.Cu" "B.Cu") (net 1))
 (segment (start 100.33 99.726893) (end 100.33 101.1936) (width 0.4) (layer "B.Cu") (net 1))
 (segment (start 100.273821 99.670714) (end 100.33 99.726893) (width 0.4) (layer "B.Cu") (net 1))
 (segment (start 100.33 101.1936) (end 99.474959 102.048641) (width 0.4) (layer "B.Cu") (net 1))
 (segment (start 100.415999 103.379999) (end 100.415999 101.787599) (width 0.4) (layer "F.Cu") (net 4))
 (segment (start 99.416 100.7876) (end 99.416 99.058001) (width 0.4) (layer "F.Cu") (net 4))
 (segment (start 100.415999 101.787599) (end 99.416 100.7876) (width 0.4) (layer "F.Cu") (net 4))
 (segment (start 104.144 107.187999) (end 104.144 103.377999) (width 0.2) (layer "F.Cu") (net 5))
 (segment (start 96.1644 102.717599) (end 96.1644 99.466401) (width 0.2) (layer "F.Cu") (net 5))
 (segment (start 95.504 107.187999) (end 95.504 103.377999) (width 0.2) (layer "F.Cu") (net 5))
 (segment (start 96.1644 99.466401) (end 95.504 98.806001) (width 0.2) (layer "F.Cu") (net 5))
 (segment (start 103.523197 99.426804) (end 104.144 98.806001) (width 0.2) (layer "F.Cu") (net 5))
 (segment (start 95.504 103.377999) (end 96.1644 102.717599) (width 0.2) (layer "F.Cu") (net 5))
 (segment (start 104.144 103.377999) (end 103.523197 102.757196) (width 0.2) (layer "F.Cu") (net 5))
 (segment (start 95.504 98.806001) (end 95.504 94.996001) (width 0.2) (layer "F.Cu") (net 5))
 (segment (start 95.504 94.996001) (end 104.144 94.996001) (width 0.2) (layer "F.Cu") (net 5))
 (segment (start 95.504 107.187999) (end 104.144 107.187999) (width 0.2) (layer "F.Cu") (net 5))
 (segment (start 104.144 98.806001) (end 104.144 94.996001) (width 0.2) (layer "F.Cu") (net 5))
 (segment (start 103.523197 102.757196) (end 103.523197 99.426804) (width 0.2) (layer "F.Cu") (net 5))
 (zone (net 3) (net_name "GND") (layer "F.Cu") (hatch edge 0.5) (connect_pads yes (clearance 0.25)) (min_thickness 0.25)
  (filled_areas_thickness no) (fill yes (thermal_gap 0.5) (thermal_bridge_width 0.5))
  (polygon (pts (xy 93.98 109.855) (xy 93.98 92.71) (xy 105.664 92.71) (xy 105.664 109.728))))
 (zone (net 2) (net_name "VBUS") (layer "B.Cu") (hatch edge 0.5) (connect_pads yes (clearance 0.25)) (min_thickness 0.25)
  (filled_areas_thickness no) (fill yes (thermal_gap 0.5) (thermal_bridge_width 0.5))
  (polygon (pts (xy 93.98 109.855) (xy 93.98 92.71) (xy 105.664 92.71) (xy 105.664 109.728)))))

